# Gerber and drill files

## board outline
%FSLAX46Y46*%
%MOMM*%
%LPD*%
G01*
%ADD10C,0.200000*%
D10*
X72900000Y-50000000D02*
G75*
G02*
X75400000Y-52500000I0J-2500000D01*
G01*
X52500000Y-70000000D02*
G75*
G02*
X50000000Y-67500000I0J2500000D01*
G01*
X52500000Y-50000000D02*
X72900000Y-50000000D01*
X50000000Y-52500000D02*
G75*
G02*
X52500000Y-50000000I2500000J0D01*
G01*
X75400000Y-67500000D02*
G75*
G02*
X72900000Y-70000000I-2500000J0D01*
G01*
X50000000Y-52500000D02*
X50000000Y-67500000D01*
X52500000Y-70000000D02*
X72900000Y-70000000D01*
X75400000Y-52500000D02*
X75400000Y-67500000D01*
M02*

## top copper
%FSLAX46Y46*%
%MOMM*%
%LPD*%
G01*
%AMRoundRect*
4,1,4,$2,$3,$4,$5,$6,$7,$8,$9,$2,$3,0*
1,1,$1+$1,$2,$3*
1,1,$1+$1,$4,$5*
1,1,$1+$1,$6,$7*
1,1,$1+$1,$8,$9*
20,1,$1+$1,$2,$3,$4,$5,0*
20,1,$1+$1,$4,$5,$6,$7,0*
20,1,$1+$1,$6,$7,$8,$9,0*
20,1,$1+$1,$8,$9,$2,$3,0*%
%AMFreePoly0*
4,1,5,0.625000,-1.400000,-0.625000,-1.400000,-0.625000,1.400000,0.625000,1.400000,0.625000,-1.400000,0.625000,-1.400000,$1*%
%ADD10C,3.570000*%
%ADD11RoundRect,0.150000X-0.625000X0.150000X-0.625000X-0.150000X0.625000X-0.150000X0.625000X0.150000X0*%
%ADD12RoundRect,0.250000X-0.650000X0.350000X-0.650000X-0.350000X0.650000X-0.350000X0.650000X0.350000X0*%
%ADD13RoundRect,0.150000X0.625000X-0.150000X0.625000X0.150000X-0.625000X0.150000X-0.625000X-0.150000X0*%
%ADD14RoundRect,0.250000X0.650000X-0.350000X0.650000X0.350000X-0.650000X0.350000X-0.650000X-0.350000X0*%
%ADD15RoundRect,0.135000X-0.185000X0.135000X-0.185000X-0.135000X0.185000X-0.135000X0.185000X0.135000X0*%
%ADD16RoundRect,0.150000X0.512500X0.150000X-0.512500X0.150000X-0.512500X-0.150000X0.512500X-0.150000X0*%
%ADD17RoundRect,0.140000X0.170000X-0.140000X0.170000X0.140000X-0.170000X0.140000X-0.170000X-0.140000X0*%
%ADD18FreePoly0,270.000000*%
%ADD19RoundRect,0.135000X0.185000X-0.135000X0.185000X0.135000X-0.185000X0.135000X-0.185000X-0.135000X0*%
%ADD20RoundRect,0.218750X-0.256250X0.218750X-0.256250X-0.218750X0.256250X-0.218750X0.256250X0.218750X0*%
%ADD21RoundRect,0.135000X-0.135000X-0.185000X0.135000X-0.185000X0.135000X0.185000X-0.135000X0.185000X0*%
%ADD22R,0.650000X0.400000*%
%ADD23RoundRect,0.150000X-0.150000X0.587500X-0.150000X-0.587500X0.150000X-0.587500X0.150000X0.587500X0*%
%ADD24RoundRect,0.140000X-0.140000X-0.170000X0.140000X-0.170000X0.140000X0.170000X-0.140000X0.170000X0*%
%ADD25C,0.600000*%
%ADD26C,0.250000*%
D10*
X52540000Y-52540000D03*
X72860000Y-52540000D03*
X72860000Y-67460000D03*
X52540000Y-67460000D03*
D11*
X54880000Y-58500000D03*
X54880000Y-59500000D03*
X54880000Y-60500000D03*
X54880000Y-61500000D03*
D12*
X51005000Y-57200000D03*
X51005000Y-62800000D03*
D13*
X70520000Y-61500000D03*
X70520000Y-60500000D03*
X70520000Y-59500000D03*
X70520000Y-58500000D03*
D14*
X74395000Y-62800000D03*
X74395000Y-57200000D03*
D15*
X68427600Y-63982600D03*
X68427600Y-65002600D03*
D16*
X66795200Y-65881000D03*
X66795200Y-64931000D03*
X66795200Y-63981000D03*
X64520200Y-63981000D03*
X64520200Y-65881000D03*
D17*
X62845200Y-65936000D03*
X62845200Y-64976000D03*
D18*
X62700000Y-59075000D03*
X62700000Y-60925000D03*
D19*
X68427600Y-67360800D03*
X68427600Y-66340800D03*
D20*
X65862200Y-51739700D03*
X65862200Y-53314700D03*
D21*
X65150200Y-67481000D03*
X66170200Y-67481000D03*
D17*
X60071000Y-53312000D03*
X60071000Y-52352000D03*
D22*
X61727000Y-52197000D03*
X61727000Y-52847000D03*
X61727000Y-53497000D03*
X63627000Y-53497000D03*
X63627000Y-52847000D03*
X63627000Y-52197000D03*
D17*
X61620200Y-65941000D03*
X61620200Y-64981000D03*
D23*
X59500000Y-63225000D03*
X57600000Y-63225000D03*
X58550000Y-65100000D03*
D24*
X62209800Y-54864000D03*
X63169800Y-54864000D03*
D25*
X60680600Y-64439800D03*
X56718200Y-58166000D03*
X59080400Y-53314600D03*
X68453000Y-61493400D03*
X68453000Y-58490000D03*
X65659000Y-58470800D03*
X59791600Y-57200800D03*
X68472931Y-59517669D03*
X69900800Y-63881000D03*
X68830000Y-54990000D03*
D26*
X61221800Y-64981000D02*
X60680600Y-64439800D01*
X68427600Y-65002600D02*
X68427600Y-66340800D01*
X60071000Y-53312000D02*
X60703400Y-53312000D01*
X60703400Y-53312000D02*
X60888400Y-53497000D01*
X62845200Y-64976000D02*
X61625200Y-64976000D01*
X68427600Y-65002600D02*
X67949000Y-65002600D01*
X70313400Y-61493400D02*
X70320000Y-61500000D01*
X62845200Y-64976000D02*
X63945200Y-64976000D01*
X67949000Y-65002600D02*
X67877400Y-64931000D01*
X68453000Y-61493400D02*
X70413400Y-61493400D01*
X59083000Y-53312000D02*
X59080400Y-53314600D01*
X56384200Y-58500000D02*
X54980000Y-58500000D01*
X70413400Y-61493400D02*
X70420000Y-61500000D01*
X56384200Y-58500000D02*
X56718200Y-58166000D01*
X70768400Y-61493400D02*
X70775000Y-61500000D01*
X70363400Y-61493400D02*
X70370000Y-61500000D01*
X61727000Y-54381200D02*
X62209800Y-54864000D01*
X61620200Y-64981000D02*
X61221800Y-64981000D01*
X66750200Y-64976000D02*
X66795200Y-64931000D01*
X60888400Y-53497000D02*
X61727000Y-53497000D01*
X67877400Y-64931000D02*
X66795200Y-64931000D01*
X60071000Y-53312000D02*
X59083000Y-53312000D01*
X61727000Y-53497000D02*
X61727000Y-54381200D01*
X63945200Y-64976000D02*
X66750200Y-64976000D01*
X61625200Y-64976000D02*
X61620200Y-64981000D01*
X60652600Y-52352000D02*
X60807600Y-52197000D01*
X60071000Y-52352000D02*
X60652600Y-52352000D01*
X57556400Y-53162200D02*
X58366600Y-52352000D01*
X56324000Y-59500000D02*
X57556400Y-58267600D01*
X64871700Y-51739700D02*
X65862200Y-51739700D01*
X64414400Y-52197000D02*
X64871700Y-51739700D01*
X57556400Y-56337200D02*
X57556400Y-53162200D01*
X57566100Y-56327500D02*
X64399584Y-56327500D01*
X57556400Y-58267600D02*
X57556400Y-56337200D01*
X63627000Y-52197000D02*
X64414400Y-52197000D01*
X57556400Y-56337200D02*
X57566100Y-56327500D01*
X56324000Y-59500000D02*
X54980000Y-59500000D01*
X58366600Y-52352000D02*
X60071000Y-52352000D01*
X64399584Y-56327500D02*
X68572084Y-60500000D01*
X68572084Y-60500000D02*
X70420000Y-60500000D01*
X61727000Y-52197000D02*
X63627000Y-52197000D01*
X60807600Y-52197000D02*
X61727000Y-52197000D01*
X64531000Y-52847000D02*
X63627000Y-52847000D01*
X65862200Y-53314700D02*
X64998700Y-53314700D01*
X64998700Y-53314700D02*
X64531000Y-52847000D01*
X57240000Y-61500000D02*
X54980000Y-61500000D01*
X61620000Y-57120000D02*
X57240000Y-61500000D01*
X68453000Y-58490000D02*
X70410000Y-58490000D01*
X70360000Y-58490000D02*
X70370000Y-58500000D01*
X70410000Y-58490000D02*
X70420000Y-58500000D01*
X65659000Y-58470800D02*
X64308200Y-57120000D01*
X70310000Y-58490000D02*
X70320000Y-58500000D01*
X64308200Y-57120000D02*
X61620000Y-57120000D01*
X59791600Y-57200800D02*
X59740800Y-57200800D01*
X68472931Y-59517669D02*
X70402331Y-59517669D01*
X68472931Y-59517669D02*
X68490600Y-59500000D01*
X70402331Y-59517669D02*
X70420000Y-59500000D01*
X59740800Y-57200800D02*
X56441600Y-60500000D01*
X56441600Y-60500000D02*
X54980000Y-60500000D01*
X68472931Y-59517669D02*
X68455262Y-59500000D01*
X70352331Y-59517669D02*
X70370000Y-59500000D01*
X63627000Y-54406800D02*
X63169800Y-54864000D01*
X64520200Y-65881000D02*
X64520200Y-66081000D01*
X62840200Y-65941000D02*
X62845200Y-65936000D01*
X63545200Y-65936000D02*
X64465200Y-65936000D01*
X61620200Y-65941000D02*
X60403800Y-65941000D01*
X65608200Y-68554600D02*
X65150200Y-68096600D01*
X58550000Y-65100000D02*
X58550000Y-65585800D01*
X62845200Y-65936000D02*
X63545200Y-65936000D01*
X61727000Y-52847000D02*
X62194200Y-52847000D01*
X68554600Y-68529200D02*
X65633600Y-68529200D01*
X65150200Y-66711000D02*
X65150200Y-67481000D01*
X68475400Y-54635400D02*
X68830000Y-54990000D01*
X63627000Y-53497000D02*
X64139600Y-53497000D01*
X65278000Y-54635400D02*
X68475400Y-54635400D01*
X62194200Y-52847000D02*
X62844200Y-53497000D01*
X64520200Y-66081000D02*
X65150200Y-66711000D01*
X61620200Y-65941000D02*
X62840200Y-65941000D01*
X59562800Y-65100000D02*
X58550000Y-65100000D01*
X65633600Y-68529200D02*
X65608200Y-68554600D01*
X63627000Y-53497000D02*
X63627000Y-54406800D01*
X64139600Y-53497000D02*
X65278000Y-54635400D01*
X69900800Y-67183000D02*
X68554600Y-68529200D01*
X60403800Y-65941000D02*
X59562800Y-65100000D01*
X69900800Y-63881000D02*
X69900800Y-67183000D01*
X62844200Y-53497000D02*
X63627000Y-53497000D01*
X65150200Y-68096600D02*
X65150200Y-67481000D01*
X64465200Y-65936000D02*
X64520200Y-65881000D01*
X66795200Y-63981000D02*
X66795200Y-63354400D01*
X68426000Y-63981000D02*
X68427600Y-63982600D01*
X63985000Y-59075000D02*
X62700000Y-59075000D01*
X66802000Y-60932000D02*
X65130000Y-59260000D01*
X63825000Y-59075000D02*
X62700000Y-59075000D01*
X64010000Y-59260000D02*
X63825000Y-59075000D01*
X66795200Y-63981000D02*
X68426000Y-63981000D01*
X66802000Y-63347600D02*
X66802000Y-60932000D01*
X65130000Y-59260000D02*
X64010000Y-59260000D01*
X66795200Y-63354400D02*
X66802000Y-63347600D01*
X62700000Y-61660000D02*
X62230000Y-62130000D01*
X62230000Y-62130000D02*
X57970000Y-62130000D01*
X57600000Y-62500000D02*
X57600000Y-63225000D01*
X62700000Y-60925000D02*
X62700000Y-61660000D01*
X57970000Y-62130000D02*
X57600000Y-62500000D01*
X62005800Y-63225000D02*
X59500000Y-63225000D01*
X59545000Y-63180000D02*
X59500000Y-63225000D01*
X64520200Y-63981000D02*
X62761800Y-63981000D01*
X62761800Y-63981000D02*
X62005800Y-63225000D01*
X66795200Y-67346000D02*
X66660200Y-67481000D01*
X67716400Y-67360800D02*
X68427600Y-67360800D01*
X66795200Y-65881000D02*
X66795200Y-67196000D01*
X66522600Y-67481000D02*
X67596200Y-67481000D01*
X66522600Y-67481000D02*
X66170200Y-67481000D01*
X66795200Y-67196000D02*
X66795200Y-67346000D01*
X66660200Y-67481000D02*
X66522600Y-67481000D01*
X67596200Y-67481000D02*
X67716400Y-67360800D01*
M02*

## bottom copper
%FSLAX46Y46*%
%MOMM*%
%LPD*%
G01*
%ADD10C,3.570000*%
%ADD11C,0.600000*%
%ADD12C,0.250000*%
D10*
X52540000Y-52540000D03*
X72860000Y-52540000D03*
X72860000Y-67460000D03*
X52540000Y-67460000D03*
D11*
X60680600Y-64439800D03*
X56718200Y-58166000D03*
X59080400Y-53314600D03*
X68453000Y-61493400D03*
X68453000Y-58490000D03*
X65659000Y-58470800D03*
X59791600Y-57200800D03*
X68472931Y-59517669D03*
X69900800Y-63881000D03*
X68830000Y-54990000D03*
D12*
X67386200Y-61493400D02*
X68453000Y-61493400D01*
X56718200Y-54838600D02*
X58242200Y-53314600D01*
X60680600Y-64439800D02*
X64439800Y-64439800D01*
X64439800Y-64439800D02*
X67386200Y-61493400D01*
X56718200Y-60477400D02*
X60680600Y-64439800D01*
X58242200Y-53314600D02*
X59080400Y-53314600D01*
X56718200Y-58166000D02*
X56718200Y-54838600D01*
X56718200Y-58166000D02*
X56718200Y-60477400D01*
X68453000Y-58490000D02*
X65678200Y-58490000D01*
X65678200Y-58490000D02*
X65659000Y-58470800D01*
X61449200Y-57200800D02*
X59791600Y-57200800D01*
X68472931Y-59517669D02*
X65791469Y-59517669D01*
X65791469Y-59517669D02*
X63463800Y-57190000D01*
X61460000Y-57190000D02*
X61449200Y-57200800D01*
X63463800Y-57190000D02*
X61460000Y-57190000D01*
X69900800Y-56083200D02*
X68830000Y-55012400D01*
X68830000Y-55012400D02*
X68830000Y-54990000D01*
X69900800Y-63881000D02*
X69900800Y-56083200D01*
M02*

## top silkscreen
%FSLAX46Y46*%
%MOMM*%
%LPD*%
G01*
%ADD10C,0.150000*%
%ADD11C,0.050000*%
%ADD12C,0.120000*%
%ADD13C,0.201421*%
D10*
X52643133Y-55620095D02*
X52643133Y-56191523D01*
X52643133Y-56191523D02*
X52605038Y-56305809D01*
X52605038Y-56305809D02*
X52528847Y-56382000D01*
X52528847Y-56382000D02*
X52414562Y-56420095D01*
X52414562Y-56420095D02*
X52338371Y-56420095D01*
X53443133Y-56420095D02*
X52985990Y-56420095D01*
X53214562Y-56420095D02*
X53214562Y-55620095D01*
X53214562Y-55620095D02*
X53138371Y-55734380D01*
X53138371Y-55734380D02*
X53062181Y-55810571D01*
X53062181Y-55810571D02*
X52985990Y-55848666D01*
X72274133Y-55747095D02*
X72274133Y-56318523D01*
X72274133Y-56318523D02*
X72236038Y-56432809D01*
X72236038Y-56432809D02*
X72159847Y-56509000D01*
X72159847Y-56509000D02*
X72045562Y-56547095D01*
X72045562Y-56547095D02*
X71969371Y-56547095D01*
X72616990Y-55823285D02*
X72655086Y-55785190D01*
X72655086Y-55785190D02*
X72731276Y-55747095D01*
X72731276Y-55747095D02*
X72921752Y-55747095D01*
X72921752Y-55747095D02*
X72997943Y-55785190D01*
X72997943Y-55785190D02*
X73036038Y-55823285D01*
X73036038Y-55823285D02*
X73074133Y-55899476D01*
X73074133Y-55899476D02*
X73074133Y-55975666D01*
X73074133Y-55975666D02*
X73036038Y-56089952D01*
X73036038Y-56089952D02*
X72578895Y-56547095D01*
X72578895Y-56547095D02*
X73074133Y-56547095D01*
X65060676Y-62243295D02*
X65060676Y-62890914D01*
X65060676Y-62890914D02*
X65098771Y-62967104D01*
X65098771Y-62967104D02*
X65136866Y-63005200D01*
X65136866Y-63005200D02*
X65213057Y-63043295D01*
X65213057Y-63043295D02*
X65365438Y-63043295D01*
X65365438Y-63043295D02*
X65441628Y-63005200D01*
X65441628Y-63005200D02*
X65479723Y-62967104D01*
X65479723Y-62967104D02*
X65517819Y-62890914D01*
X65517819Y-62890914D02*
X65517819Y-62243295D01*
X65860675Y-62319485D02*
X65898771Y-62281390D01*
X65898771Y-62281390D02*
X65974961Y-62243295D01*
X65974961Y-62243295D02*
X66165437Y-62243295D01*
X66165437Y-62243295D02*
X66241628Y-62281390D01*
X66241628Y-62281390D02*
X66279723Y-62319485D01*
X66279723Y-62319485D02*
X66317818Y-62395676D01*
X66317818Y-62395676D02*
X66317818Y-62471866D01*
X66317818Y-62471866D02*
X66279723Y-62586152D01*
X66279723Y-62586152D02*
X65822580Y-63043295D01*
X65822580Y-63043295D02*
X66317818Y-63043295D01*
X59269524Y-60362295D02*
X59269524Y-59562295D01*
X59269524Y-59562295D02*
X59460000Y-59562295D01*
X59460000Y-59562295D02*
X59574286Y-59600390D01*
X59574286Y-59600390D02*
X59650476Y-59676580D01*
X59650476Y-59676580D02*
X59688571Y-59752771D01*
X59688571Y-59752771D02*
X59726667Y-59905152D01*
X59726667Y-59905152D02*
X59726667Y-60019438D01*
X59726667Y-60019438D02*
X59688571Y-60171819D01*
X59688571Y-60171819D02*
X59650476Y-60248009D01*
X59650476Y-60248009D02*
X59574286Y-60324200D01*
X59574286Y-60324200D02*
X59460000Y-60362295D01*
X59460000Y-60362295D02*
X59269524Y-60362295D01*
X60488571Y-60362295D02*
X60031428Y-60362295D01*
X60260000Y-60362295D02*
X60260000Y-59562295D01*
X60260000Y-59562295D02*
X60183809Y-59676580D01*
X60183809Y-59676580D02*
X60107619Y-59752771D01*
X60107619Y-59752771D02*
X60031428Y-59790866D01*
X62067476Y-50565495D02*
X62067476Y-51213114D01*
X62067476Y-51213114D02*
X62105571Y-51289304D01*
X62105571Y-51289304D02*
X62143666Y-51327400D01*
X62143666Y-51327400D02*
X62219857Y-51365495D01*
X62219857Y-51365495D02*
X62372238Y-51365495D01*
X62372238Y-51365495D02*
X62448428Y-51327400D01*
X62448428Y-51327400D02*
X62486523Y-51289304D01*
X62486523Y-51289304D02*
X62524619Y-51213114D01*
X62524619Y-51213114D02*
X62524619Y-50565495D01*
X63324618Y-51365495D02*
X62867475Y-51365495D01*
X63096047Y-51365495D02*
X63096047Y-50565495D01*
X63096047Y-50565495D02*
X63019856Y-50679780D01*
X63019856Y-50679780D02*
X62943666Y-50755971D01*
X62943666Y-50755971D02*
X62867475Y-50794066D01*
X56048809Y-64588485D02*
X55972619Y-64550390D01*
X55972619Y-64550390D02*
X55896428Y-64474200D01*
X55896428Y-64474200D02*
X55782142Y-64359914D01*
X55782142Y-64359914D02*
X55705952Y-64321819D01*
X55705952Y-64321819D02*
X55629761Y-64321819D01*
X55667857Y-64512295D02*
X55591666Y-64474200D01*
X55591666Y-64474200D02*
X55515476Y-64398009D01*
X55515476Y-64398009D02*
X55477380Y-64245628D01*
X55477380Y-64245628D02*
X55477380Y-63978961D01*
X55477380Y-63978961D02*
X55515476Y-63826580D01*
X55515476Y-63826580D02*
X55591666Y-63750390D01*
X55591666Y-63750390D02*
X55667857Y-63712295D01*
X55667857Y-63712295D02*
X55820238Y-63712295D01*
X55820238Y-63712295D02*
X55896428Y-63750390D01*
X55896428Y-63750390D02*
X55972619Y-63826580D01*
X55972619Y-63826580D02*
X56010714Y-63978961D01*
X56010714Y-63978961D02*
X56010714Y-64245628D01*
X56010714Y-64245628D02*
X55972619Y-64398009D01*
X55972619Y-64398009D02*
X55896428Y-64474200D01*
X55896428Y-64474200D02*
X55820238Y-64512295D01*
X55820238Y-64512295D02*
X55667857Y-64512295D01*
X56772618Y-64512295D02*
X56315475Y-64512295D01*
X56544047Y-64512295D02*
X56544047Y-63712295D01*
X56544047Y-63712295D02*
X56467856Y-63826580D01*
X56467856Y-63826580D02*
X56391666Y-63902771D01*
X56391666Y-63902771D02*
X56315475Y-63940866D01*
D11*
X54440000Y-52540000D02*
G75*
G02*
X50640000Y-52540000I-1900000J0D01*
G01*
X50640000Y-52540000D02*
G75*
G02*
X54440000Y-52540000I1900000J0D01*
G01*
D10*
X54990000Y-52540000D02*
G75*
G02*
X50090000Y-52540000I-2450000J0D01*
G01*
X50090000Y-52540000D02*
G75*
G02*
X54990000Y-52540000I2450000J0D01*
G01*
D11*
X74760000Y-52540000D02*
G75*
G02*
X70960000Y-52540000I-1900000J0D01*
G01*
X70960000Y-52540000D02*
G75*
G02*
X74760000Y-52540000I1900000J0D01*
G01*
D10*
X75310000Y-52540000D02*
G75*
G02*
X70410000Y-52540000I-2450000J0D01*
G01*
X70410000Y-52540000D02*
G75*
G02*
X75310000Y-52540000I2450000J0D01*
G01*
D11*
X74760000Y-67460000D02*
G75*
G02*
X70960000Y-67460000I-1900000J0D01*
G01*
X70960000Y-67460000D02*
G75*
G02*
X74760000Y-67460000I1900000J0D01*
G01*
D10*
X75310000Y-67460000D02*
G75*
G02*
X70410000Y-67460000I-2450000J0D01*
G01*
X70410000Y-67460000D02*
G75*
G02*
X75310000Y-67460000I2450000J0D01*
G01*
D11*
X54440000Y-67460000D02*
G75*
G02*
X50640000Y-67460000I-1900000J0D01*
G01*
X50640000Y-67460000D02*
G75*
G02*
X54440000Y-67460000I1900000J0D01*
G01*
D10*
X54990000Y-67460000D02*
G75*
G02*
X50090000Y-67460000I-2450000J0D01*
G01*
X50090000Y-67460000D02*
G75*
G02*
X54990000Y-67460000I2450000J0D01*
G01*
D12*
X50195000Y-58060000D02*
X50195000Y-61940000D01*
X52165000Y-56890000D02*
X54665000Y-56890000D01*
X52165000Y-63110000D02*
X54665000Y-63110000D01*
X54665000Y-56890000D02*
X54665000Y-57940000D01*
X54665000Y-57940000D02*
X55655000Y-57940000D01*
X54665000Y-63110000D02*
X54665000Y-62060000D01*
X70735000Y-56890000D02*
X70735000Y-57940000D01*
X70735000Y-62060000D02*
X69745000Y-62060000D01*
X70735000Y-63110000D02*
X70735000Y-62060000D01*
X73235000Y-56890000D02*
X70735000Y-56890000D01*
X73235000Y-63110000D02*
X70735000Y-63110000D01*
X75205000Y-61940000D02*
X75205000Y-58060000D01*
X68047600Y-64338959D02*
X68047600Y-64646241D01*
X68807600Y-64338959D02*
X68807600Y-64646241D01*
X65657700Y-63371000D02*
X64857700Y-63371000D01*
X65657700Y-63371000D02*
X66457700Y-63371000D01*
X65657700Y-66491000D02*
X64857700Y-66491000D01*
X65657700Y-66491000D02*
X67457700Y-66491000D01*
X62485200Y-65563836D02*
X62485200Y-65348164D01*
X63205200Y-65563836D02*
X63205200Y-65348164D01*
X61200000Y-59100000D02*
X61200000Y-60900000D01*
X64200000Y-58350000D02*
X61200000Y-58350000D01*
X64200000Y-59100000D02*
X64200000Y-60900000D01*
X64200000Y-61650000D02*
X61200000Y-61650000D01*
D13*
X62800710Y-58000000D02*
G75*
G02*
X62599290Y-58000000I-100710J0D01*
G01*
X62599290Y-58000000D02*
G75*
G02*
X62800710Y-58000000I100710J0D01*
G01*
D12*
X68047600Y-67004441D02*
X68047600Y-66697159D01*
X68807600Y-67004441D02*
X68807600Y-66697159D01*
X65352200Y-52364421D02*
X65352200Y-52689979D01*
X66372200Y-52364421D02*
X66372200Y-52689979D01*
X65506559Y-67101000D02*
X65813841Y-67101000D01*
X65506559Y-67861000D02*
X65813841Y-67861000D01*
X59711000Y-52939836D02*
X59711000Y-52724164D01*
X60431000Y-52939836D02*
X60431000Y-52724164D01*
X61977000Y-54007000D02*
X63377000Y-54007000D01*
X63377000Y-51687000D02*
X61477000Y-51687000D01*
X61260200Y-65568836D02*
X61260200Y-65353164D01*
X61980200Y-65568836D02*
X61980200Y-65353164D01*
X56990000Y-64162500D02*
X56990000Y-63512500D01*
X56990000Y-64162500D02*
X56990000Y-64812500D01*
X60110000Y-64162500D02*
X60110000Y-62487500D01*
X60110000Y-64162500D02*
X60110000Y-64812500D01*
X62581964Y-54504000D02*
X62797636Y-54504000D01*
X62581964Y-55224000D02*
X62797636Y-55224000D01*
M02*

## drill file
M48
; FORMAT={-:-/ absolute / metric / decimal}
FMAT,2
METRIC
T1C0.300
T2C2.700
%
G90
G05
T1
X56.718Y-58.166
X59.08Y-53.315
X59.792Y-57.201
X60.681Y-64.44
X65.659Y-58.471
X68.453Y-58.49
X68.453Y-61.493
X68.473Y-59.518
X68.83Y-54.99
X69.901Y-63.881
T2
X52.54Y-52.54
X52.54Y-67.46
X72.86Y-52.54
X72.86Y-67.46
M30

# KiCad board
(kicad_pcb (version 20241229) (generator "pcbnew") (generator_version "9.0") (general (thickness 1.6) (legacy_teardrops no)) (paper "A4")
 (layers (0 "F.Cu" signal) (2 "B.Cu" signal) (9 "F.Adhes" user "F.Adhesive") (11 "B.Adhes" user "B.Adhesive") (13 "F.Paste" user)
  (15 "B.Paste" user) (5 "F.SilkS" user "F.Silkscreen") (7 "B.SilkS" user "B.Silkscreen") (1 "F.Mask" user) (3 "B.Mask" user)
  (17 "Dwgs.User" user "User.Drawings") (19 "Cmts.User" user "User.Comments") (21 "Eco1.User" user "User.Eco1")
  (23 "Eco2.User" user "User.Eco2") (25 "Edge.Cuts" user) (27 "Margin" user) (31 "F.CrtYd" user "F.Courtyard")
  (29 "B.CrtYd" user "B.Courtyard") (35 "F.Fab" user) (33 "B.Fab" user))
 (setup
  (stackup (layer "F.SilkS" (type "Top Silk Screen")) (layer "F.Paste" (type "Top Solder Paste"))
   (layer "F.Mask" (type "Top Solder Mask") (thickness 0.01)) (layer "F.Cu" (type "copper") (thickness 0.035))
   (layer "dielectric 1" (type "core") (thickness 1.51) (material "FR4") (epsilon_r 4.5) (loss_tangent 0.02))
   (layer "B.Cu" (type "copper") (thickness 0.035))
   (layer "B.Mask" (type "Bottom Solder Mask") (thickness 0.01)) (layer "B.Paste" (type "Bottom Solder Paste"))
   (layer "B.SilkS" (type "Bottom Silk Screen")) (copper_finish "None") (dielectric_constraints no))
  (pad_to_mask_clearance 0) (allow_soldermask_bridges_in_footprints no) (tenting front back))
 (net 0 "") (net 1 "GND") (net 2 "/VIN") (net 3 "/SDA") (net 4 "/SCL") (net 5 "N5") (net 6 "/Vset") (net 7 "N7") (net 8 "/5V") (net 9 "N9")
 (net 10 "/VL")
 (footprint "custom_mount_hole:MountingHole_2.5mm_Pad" (layer "F.Cu") (at 52.54 52.54)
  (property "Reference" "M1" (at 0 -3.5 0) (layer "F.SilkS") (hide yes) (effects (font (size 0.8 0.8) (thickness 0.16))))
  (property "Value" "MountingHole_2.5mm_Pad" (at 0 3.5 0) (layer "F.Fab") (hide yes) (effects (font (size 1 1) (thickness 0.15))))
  (fp_circle (center 0 0) (end 1.9 0) (stroke (width 0.05) (type solid)) (fill no) (layer "F.SilkS"))
  (fp_circle (center 0 0) (end 2.45 0) (stroke (width 0.15) (type solid)) (fill no) (layer "F.SilkS"))
  (pad "~" thru_hole circle (at 0 0) (size 3.57 3.57) (drill 2.7) (layers "*.Cu" "*.Mask") (remove_unused_layers no)))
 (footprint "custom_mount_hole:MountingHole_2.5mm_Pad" (layer "F.Cu") (at 72.86 52.54)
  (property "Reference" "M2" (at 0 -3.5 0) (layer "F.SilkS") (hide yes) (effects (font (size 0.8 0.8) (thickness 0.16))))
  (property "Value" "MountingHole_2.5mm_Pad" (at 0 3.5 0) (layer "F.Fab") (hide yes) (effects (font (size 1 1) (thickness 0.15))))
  (fp_circle (center 0 0) (end 1.9 0) (stroke (width 0.05) (type solid)) (fill no) (layer "F.SilkS"))
  (fp_circle (center 0 0) (end 2.45 0) (stroke (width 0.15) (type solid)) (fill no) (layer "F.SilkS"))
  (pad "~" thru_hole circle (at 0 0) (size 3.57 3.57) (drill 2.7) (layers "*.Cu" "*.Mask") (remove_unused_layers no)))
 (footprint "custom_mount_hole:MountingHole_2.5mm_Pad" (layer "F.Cu") (at 72.86 67.46)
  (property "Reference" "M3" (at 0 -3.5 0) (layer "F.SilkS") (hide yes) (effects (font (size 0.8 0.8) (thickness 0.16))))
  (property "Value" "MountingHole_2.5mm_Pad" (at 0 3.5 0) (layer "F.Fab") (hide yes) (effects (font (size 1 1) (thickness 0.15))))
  (fp_circle (center 0 0) (end 1.9 0) (stroke (width 0.05) (type solid)) (fill no) (layer "F.SilkS"))
  (fp_circle (center 0 0) (end 2.45 0) (stroke (width 0.15) (type solid)) (fill no) (layer "F.SilkS"))
  (pad "~" thru_hole circle (at 0 0) (size 3.57 3.57) (drill 2.7) (layers "*.Cu" "*.Mask") (remove_unused_layers no)))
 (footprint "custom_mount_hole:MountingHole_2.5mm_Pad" (layer "F.Cu") (at 52.54 67.46)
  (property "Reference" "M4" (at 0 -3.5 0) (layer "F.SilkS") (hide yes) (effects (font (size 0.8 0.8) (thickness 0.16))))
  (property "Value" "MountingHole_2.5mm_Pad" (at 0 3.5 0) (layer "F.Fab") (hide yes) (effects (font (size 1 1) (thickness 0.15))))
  (fp_circle (center 0 0) (end 1.9 0) (stroke (width 0.05) (type solid)) (fill no) (layer "F.SilkS"))
  (fp_circle (center 0 0) (end 2.45 0) (stroke (width 0.15) (type solid)) (fill no) (layer "F.SilkS"))
  (pad "~" thru_hole circle (at 0 0) (size 3.57 3.57) (drill 2.7) (layers "*.Cu" "*.Mask") (remove_unused_layers no)))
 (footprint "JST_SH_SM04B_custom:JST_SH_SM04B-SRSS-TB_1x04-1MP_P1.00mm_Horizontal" (layer "F.Cu") (at 52.88 60 -90)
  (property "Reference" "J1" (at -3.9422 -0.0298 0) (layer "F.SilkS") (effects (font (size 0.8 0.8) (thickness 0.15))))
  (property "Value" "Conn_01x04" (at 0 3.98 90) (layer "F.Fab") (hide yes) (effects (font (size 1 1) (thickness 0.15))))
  (fp_line (start -1.94 2.685) (end 1.94 2.685) (stroke (width 0.12) (type solid)) (layer "F.SilkS"))
  (fp_line (start -3.11 0.715) (end -3.11 -1.785) (stroke (width 0.12) (type solid)) (layer "F.SilkS"))
  (fp_line (start 3.11 0.715) (end 3.11 -1.785) (stroke (width 0.12) (type solid)) (layer "F.SilkS"))
  (fp_line (start -3.11 -1.785) (end -2.06 -1.785) (stroke (width 0.12) (type solid)) (layer "F.SilkS"))
  (fp_line (start -2.06 -1.785) (end -2.06 -2.775) (stroke (width 0.12) (type solid)) (layer "F.SilkS"))
  (fp_line (start 3.11 -1.785) (end 2.06 -1.785) (stroke (width 0.12) (type solid)) (layer "F.SilkS"))
  (pad "1" smd roundrect (at -1.5 -2 270) (size 0.6 1.55) (layers "F.Cu" "F.Mask" "F.Paste") (roundrect_rratio 0.25) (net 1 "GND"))
  (pad "2" smd roundrect (at -0.5 -2 270) (size 0.6 1.55) (layers "F.Cu" "F.Mask" "F.Paste") (roundrect_rratio 0.25) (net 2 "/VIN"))
  (pad "3" smd roundrect (at 0.5 -2 270) (size 0.6 1.55) (layers "F.Cu" "F.Mask" "F.Paste") (roundrect_rratio 0.25) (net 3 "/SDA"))
  (pad "4" smd roundrect (at 1.5 -2 270) (size 0.6 1.55) (layers "F.Cu" "F.Mask" "F.Paste") (roundrect_rratio 0.25) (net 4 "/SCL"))
  (pad "MP" smd roundrect (at -2.8 1.875 270) (size 1.2 1.8) (layers "F.Cu" "F.Mask" "F.Paste") (roundrect_rratio 0.2083333333))
  (pad "MP" smd roundrect (at 2.8 1.875 270) (size 1.2 1.8) (layers "F.Cu" "F.Mask" "F.Paste") (roundrect_rratio 0.2083333333)))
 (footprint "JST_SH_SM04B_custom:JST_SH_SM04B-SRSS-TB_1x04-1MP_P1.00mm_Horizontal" (layer "F.Cu") (at 72.52 60 90)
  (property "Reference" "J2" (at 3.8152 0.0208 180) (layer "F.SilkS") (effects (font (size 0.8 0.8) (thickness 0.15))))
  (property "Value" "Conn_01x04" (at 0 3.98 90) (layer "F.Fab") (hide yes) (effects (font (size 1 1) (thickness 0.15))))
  (fp_line (start 3.11 -1.785) (end 2.06 -1.785) (stroke (width 0.12) (type solid)) (layer "F.SilkS"))
  (fp_line (start -2.06 -1.785) (end -2.06 -2.775) (stroke (width 0.12) (type solid)) (layer "F.SilkS"))
  (fp_line (start -3.11 -1.785) (end -2.06 -1.785) (stroke (width 0.12) (type solid)) (layer "F.SilkS"))
  (fp_line (start 3.11 0.715) (end 3.11 -1.785) (stroke (width 0.12) (type solid)) (layer "F.SilkS"))
  (fp_line (start -3.11 0.715) (end -3.11 -1.785) (stroke (width 0.12) (type solid)) (layer "F.SilkS"))
  (fp_line (start -1.94 2.685) (end 1.94 2.685) (stroke (width 0.12) (type solid)) (layer "F.SilkS"))
  (pad "1" smd roundrect (at -1.5 -2 90) (size 0.6 1.55) (layers "F.Cu" "F.Mask" "F.Paste") (roundrect_rratio 0.25) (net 1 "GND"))
  (pad "2" smd roundrect (at -0.5 -2 90) (size 0.6 1.55) (layers "F.Cu" "F.Mask" "F.Paste") (roundrect_rratio 0.25) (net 2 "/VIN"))
  (pad "3" smd roundrect (at 0.5 -2 90) (size 0.6 1.55) (layers "F.Cu" "F.Mask" "F.Paste") (roundrect_rratio 0.25) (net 3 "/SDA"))
  (pad "4" smd roundrect (at 1.5 -2 90) (size 0.6 1.55) (layers "F.Cu" "F.Mask" "F.Paste") (roundrect_rratio 0.25) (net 4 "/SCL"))
  (pad "MP" smd roundrect (at -2.8 1.875 90) (size 1.2 1.8) (layers "F.Cu" "F.Mask" "F.Paste") (roundrect_rratio 0.2083333333))
  (pad "MP" smd roundrect (at 2.8 1.875 90) (size 1.2 1.8) (layers "F.Cu" "F.Mask" "F.Paste") (roundrect_rratio 0.2083333333)))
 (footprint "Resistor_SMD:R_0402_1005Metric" (layer "F.Cu") (at 68.4276 64.4926 -90)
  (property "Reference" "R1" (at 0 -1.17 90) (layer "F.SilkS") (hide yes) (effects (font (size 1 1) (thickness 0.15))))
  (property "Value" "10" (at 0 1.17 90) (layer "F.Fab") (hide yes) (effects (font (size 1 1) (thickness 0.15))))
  (fp_line (start -0.153641 0.38) (end 0.153641 0.38) (stroke (width 0.12) (type solid)) (layer "F.SilkS"))
  (fp_line (start -0.153641 -0.38) (end 0.153641 -0.38) (stroke (width 0.12) (type solid)) (layer "F.SilkS"))
  (pad "1" smd roundrect (at -0.51 0 270) (size 0.54 0.64) (layers "F.Cu" "F.Mask" "F.Paste") (roundrect_rratio 0.25) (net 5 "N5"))
  (pad "2" smd roundrect (at 0.51 0 270) (size 0.54 0.64) (layers "F.Cu" "F.Mask" "F.Paste") (roundrect_rratio 0.25) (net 1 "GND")))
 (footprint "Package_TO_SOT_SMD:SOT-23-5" (layer "F.Cu") (at 65.6577 64.931 180)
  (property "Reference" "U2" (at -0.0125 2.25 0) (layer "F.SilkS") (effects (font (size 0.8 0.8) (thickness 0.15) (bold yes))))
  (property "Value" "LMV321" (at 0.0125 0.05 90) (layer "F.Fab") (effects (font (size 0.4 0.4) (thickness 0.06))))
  (fp_line (start 0 1.56) (end 0.8 1.56) (stroke (width 0.12) (type solid)) (layer "F.SilkS"))
  (fp_line (start 0 1.56) (end -0.8 1.56) (stroke (width 0.12) (type solid)) (layer "F.SilkS"))
  (fp_line (start 0 -1.56) (end 0.8 -1.56) (stroke (width 0.12) (type solid)) (layer "F.SilkS"))
  (fp_line (start 0 -1.56) (end -1.8 -1.56) (stroke (width 0.12) (type solid)) (layer "F.SilkS"))
  (pad "1" smd roundrect (at -1.1375 -0.95 180) (size 1.325 0.6) (layers "F.Cu" "F.Mask" "F.Paste") (roundrect_rratio 0.25) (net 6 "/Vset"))
  (pad "2" smd roundrect (at -1.1375 0 180) (size 1.325 0.6) (layers "F.Cu" "F.Mask" "F.Paste") (roundrect_rratio 0.25) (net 1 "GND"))
  (pad "3" smd roundrect (at -1.1375 0.95 180) (size 1.325 0.6) (layers "F.Cu" "F.Mask" "F.Paste") (roundrect_rratio 0.25) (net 5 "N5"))
  (pad "4" smd roundrect (at 1.1375 0.95 180) (size 1.325 0.6) (layers "F.Cu" "F.Mask" "F.Paste") (roundrect_rratio 0.25) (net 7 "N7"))
  (pad "5" smd roundrect (at 1.1375 -0.95 180) (size 1.325 0.6) (layers "F.Cu" "F.Mask" "F.Paste") (roundrect_rratio 0.25) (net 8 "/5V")))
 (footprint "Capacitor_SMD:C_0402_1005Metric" (layer "F.Cu") (at 62.8452 65.456 90)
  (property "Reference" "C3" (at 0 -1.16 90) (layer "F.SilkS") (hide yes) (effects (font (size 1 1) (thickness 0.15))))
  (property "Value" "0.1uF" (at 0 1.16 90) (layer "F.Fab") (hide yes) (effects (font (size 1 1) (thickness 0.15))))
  (fp_line (start -0.107836 -0.36) (end 0.107836 -0.36) (stroke (width 0.12) (type solid)) (layer "F.SilkS"))
  (fp_line (start -0.107836 0.36) (end 0.107836 0.36) (stroke (width 0.12) (type solid)) (layer "F.SilkS"))
  (pad "1" smd roundrect (at -0.48 0 90) (size 0.56 0.62) (layers "F.Cu" "F.Mask" "F.Paste") (roundrect_rratio 0.25) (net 8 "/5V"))
  (pad "2" smd roundrect (at 0.48 0 90) (size 0.56 0.62) (layers "F.Cu" "F.Mask" "F.Paste") (roundrect_rratio 0.25) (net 1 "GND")))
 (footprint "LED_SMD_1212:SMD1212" (layer "F.Cu") (at 62.7 60 -90)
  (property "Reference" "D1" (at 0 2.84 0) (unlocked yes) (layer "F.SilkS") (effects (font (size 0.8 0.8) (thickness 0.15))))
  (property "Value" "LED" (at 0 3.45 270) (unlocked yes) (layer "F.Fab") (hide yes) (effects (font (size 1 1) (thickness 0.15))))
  (fp_line (start -0.9 1.5) (end 0.9 1.5) (stroke (width 0.12) (type default)) (layer "F.SilkS"))
  (fp_line (start -1.65 -1.5) (end -1.65 1.5) (stroke (width 0.12) (type default)) (layer "F.SilkS"))
  (fp_line (start -0.9 -1.5) (end 0.9 -1.5) (stroke (width 0.12) (type default)) (layer "F.SilkS"))
  (fp_line (start 1.65 -1.5) (end 1.65 1.5) (stroke (width 0.12) (type default)) (layer "F.SilkS"))
  (fp_circle (center -2 0) (end -1.9 0.1) (stroke (width 0.12) (type solid)) (fill yes) (layer "F.SilkS"))
  (pad "1" smd custom (at -0.925 0 270) (size 1.25 2.8) (layers "F.Cu" "F.Mask" "F.Paste") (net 5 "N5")
   (options (clearance outline) (anchor rect)) (primitives))
  (pad "2" smd custom (at 0.925 0 270) (size 1.25 2.8) (layers "F.Cu" "F.Mask" "F.Paste") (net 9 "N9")
   (options (clearance outline) (anchor rect)) (primitives)))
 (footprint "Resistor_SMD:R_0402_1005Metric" (layer "F.Cu") (at 68.4276 66.8508 90)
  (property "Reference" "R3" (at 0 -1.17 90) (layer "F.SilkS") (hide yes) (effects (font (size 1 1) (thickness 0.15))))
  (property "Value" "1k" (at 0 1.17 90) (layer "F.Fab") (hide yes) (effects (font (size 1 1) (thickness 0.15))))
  (fp_line (start -0.153641 -0.38) (end 0.153641 -0.38) (stroke (width 0.12) (type solid)) (layer "F.SilkS"))
  (fp_line (start -0.153641 0.38) (end 0.153641 0.38) (stroke (width 0.12) (type solid)) (layer "F.SilkS"))
  (pad "1" smd roundrect (at -0.51 0 90) (size 0.54 0.64) (layers "F.Cu" "F.Mask" "F.Paste") (roundrect_rratio 0.25) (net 6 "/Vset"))
  (pad "2" smd roundrect (at 0.51 0 90) (size 0.54 0.64) (layers "F.Cu" "F.Mask" "F.Paste") (roundrect_rratio 0.25) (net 1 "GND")))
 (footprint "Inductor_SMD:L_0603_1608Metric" (layer "F.Cu") (at 65.8622 52.5272 -90)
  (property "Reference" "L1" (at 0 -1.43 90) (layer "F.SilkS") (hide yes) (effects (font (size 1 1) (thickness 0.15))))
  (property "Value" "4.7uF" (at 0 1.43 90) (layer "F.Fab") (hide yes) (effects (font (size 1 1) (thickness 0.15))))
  (fp_line (start -0.162779 0.51) (end 0.162779 0.51) (stroke (width 0.12) (type solid)) (layer "F.SilkS"))
  (fp_line (start -0.162779 -0.51) (end 0.162779 -0.51) (stroke (width 0.12) (type solid)) (layer "F.SilkS"))
  (pad "1" smd roundrect (at -0.7875 0 270) (size 0.875 0.95) (layers "F.Cu" "F.Mask" "F.Paste") (roundrect_rratio 0.25) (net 2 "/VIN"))
  (pad "2" smd roundrect (at 0.7875 0 270) (size 0.875 0.95) (layers "F.Cu" "F.Mask" "F.Paste") (roundrect_rratio 0.25) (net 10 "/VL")))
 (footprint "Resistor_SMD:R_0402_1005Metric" (layer "F.Cu") (at 65.6602 67.481)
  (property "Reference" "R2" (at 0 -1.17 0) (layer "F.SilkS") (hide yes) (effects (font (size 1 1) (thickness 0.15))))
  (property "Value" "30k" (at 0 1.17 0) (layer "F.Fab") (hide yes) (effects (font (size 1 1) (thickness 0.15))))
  (fp_line (start -0.153641 -0.38) (end 0.153641 -0.38) (stroke (width 0.12) (type solid)) (layer "F.SilkS"))
  (fp_line (start -0.153641 0.38) (end 0.153641 0.38) (stroke (width 0.12) (type solid)) (layer "F.SilkS"))
  (pad "1" smd roundrect (at -0.51 0) (size 0.54 0.64) (layers "F.Cu" "F.Mask" "F.Paste") (roundrect_rratio 0.25) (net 8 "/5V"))
  (pad "2" smd roundrect (at 0.51 0) (size 0.54 0.64) (layers "F.Cu" "F.Mask" "F.Paste") (roundrect_rratio 0.25) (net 6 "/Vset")))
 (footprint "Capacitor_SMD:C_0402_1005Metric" (layer "F.Cu") (at 60.071 52.832 90)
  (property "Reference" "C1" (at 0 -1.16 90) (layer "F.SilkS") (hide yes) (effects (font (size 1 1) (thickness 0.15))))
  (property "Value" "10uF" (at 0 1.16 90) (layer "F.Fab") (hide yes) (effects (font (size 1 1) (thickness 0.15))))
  (fp_line (start -0.107836 -0.36) (end 0.107836 -0.36) (stroke (width 0.12) (type solid)) (layer "F.SilkS"))
  (fp_line (start -0.107836 0.36) (end 0.107836 0.36) (stroke (width 0.12) (type solid)) (layer "F.SilkS"))
  (pad "1" smd roundrect (at -0.48 0 90) (size 0.56 0.62) (layers "F.Cu" "F.Mask" "F.Paste") (roundrect_rratio 0.25) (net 1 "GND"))
  (pad "2" smd roundrect (at 0.48 0 90) (size 0.56 0.62) (layers "F.Cu" "F.Mask" "F.Paste") (roundrect_rratio 0.25) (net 2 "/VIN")))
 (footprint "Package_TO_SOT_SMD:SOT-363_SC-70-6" (layer "F.Cu") (at 62.677 52.847)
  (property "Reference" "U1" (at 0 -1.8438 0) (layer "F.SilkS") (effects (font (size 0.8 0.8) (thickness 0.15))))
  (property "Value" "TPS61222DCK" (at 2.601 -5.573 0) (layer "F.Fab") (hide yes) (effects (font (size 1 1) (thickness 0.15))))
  (fp_line (start -0.7 1.16) (end 0.7 1.16) (stroke (width 0.12) (type solid)) (layer "F.SilkS"))
  (fp_line (start 0.7 -1.16) (end -1.2 -1.16) (stroke (width 0.12) (type solid)) (layer "F.SilkS"))
  (pad "1" smd rect (at -0.95 -0.65) (size 0.65 0.4) (layers "F.Cu" "F.Mask" "F.Paste") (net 2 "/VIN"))
  (pad "2" smd rect (at -0.95 0) (size 0.65 0.4) (layers "F.Cu" "F.Mask" "F.Paste") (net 8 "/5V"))
  (pad "3" smd rect (at -0.95 0.65) (size 0.65 0.4) (layers "F.Cu" "F.Mask" "F.Paste") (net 1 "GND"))
  (pad "4" smd rect (at 0.95 0.65) (size 0.65 0.4) (layers "F.Cu" "F.Mask" "F.Paste") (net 8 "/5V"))
  (pad "5" smd rect (at 0.95 0) (size 0.65 0.4) (layers "F.Cu" "F.Mask" "F.Paste") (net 10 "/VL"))
  (pad "6" smd rect (at 0.95 -0.65) (size 0.65 0.4) (layers "F.Cu" "F.Mask" "F.Paste") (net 2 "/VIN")))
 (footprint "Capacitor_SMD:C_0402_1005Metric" (layer "F.Cu") (at 61.6202 65.461 90)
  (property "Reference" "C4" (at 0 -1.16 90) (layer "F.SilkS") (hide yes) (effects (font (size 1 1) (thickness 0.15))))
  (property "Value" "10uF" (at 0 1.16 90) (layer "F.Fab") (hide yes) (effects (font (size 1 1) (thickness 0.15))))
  (fp_line (start -0.107836 -0.36) (end 0.107836 -0.36) (stroke (width 0.12) (type solid)) (layer "F.SilkS"))
  (fp_line (start -0.107836 0.36) (end 0.107836 0.36) (stroke (width 0.12) (type solid)) (layer "F.SilkS"))
  (pad "1" smd roundrect (at -0.48 0 90) (size 0.56 0.62) (layers "F.Cu" "F.Mask" "F.Paste") (roundrect_rratio 0.25) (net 8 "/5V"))
  (pad "2" smd roundrect (at 0.48 0 90) (size 0.56 0.62) (layers "F.Cu" "F.Mask" "F.Paste") (roundrect_rratio 0.25) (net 1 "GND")))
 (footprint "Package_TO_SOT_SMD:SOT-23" (layer "F.Cu") (at 58.55 64.1625 -90)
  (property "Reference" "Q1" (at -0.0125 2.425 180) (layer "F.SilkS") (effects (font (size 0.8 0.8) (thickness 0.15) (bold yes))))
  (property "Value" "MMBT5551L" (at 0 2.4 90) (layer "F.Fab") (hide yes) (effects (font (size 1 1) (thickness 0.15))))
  (fp_line (start 0 1.56) (end -0.65 1.56) (stroke (width 0.12) (type solid)) (layer "F.SilkS"))
  (fp_line (start 0 1.56) (end 0.65 1.56) (stroke (width 0.12) (type solid)) (layer "F.SilkS"))
  (fp_line (start 0 -1.56) (end -1.675 -1.56) (stroke (width 0.12) (type solid)) (layer "F.SilkS"))
  (fp_line (start 0 -1.56) (end 0.65 -1.56) (stroke (width 0.12) (type solid)) (layer "F.SilkS"))
  (pad "1" smd roundrect (at -0.9375 -0.95 270) (size 1.475 0.6) (layers "F.Cu" "F.Mask" "F.Paste") (roundrect_rratio 0.25) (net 7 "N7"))
  (pad "2" smd roundrect (at -0.9375 0.95 270) (size 1.475 0.6) (layers "F.Cu" "F.Mask" "F.Paste") (roundrect_rratio 0.25) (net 9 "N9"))
  (pad "3" smd roundrect (at 0.9375 0 270) (size 1.475 0.6) (layers "F.Cu" "F.Mask" "F.Paste") (roundrect_rratio 0.25) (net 8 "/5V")))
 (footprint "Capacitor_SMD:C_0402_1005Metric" (layer "F.Cu") (at 62.6898 54.864)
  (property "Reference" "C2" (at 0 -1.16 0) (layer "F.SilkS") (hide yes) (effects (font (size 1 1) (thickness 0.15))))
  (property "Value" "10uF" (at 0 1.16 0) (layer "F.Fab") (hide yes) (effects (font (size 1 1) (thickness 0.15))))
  (fp_line (start -0.107836 -0.36) (end 0.107836 -0.36) (stroke (width 0.12) (type solid)) (layer "F.SilkS"))
  (fp_line (start -0.107836 0.36) (end 0.107836 0.36) (stroke (width 0.12) (type solid)) (layer "F.SilkS"))
  (pad "1" smd roundrect (at -0.48 0) (size 0.56 0.62) (layers "F.Cu" "F.Mask" "F.Paste") (roundrect_rratio 0.25) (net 1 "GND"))
  (pad "2" smd roundrect (at 0.48 0) (size 0.56 0.62) (layers "F.Cu" "F.Mask" "F.Paste") (roundrect_rratio 0.25) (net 8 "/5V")))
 (gr_arc (start 72.9 50) (mid 74.667767 50.732233) (end 75.4 52.5) (stroke (width 0.2) (type solid)) (layer "Edge.Cuts"))
 (gr_arc (start 52.5 70) (mid 50.732233 69.267767) (end 50 67.5) (stroke (width 0.2) (type solid)) (layer "Edge.Cuts"))
 (gr_line (start 52.5 50) (end 72.9 50) (stroke (width 0.2) (type solid)) (layer "Edge.Cuts"))
 (gr_arc (start 50 52.5) (mid 50.732233 50.732233) (end 52.5 50) (stroke (width 0.2) (type solid)) (layer "Edge.Cuts"))
 (gr_arc (start 75.4 67.5) (mid 74.667767 69.267767) (end 72.9 70) (stroke (width 0.2) (type solid)) (layer "Edge.Cuts"))
 (gr_line (start 50 52.5) (end 50 67.5) (stroke (width 0.2) (type solid)) (layer "Edge.Cuts"))
 (gr_line (start 52.5 70) (end 72.9 70) (stroke (width 0.2) (type solid)) (layer "Edge.Cuts"))
 (gr_line (start 75.4 52.5) (end 75.4 67.5) (stroke (width 0.2) (type solid)) (layer "Edge.Cuts"))
 (segment (start 61.2218 64.981) (end 60.6806 64.4398) (width 0.25) (layer "F.Cu") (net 1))
 (segment (start 68.4276 65.0026) (end 68.4276 66.3408) (width 0.25) (layer "F.Cu") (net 1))
 (segment (start 60.071 53.312) (end 60.7034 53.312) (width 0.25) (layer "F.Cu") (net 1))
 (segment (start 60.7034 53.312) (end 60.8884 53.497) (width 0.25) (layer "F.Cu") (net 1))
 (segment (start 62.8452 64.976) (end 61.6252 64.976) (width 0.25) (layer "F.Cu") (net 1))
 (segment (start 68.4276 65.0026) (end 67.949 65.0026) (width 0.25) (layer "F.Cu") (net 1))
 (segment (start 70.3134 61.4934) (end 70.32 61.5) (width 0.25) (layer "F.Cu") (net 1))
 (segment (start 62.8452 64.976) (end 63.9452 64.976) (width 0.25) (layer "F.Cu") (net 1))
 (segment (start 67.949 65.0026) (end 67.8774 64.931) (width 0.25) (layer "F.Cu") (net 1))
 (segment (start 68.453 61.4934) (end 70.4134 61.4934) (width 0.25) (layer "F.Cu") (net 1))
 (segment (start 59.083 53.312) (end 59.0804 53.3146) (width 0.25) (layer "F.Cu") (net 1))
 (segment (start 56.3842 58.5) (end 54.98 58.5) (width 0.25) (layer "F.Cu") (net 1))
 (segment (start 70.4134 61.4934) (end 70.42 61.5) (width 0.25) (layer "F.Cu") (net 1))
 (segment (start 56.3842 58.5) (end 56.7182 58.166) (width 0.25) (layer "F.Cu") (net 1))
 (segment (start 70.7684 61.4934) (end 70.775 61.5) (width 0.25) (layer "F.Cu") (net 1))
 (segment (start 70.3634 61.4934) (end 70.37 61.5) (width 0.25) (layer "F.Cu") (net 1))
 (segment (start 61.727 54.3812) (end 62.2098 54.864) (width 0.25) (layer "F.Cu") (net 1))
 (segment (start 61.6202 64.981) (end 61.2218 64.981) (width 0.25) (layer "F.Cu") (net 1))
 (segment (start 66.7502 64.976) (end 66.7952 64.931) (width 0.25) (layer "F.Cu") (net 1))
 (segment (start 60.8884 53.497) (end 61.727 53.497) (width 0.25) (layer "F.Cu") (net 1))
 (segment (start 67.8774 64.931) (end 66.7952 64.931) (width 0.25) (layer "F.Cu") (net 1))
 (segment (start 60.071 53.312) (end 59.083 53.312) (width 0.25) (layer "F.Cu") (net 1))
 (segment (start 61.727 53.497) (end 61.727 54.3812) (width 0.25) (layer "F.Cu") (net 1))
 (segment (start 63.9452 64.976) (end 66.7502 64.976) (width 0.25) (layer "F.Cu") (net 1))
 (segment (start 61.6252 64.976) (end 61.6202 64.981) (width 0.25) (layer "F.Cu") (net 1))
 (via (at 60.6806 64.4398) (size 0.6) (drill 0.3) (layers "F.Cu" "B.Cu") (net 1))
 (via (at 56.7182 58.166) (size 0.6) (drill 0.3) (layers "F.Cu" "B.Cu") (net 1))
 (via (at 59.0804 53.3146) (size 0.6) (drill 0.3) (layers "F.Cu" "B.Cu") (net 1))
 (via (at 68.453 61.4934) (size 0.6) (drill 0.3) (layers "F.Cu" "B.Cu") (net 1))
 (segment (start 67.3862 61.4934) (end 68.453 61.4934) (width 0.25) (layer "B.Cu") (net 1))
 (segment (start 56.7182 54.8386) (end 58.2422 53.3146) (width 0.25) (layer "B.Cu") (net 1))
 (segment (start 60.6806 64.4398) (end 64.4398 64.4398) (width 0.25) (layer "B.Cu") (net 1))
 (segment (start 64.4398 64.4398) (end 67.3862 61.4934) (width 0.25) (layer "B.Cu") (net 1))
 (segment (start 56.7182 60.4774) (end 60.6806 64.4398) (width 0.25) (layer "B.Cu") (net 1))
 (segment (start 58.2422 53.3146) (end 59.0804 53.3146) (width 0.25) (layer "B.Cu") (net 1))
 (segment (start 56.7182 58.166) (end 56.7182 54.8386) (width 0.25) (layer "B.Cu") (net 1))
 (segment (start 56.7182 58.166) (end 56.7182 60.4774) (width 0.25) (layer "B.Cu") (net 1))
 (segment (start 60.6526 52.352) (end 60.8076 52.197) (width 0.25) (layer "F.Cu") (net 2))
 (segment (start 60.071 52.352) (end 60.6526 52.352) (width 0.25) (layer "F.Cu") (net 2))
 (segment (start 57.5564 53.1622) (end 58.3666 52.352) (width 0.25) (layer "F.Cu") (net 2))
 (segment (start 56.324 59.5) (end 57.5564 58.2676) (width 0.25) (layer "F.Cu") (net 2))
 (segment (start 64.8717 51.7397) (end 65.8622 51.7397) (width 0.25) (layer "F.Cu") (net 2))
 (segment (start 64.4144 52.197) (end 64.8717 51.7397) (width 0.25) (layer "F.Cu") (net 2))
 (segment (start 57.5564 56.3372) (end 57.5564 53.1622) (width 0.25) (layer "F.Cu") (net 2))
 (segment (start 57.5661 56.3275) (end 64.399584 56.3275) (width 0.25) (layer "F.Cu") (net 2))
 (segment (start 57.5564 58.2676) (end 57.5564 56.3372) (width 0.25) (layer "F.Cu") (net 2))
 (segment (start 63.627 52.197) (end 64.4144 52.197) (width 0.25) (layer "F.Cu") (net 2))
 (segment (start 57.5564 56.3372) (end 57.5661 56.3275) (width 0.25) (layer "F.Cu") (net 2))
 (segment (start 56.324 59.5) (end 54.98 59.5) (width 0.25) (layer "F.Cu") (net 2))
 (segment (start 58.3666 52.352) (end 60.071 52.352) (width 0.25) (layer "F.Cu") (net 2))
 (segment (start 64.399584 56.3275) (end 68.572084 60.5) (width 0.25) (layer "F.Cu") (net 2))
 (segment (start 68.572084 60.5) (end 70.42 60.5) (width 0.25) (layer "F.Cu") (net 2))
 (segment (start 61.727 52.197) (end 63.627 52.197) (width 0.25) (layer "F.Cu") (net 2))
 (segment (start 60.8076 52.197) (end 61.727 52.197) (width 0.25) (layer "F.Cu") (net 2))
 (segment (start 64.531 52.847) (end 63.627 52.847) (width 0.25) (layer "F.Cu") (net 10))
 (segment (start 65.8622 53.3147) (end 64.9987 53.3147) (width 0.25) (layer "F.Cu") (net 10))
 (segment (start 64.9987 53.3147) (end 64.531 52.847) (width 0.25) (layer "F.Cu") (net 10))
 (segment (start 57.24 61.5) (end 54.98 61.5) (width 0.25) (layer "F.Cu") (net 4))
 (segment (start 61.62 57.12) (end 57.24 61.5) (width 0.25) (layer "F.Cu") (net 4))
 (segment (start 68.453 58.49) (end 70.41 58.49) (width 0.25) (layer "F.Cu") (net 4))
 (segment (start 70.36 58.49) (end 70.37 58.5) (width 0.25) (layer "F.Cu") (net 4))
 (segment (start 70.41 58.49) (end 70.42 58.5) (width 0.25) (layer "F.Cu") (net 4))
 (segment (start 65.659 58.4708) (end 64.3082 57.12) (width 0.25) (layer "F.Cu") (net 4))
 (segment (start 70.31 58.49) (end 70.32 58.5) (width 0.25) (layer "F.Cu") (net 4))
 (segment (start 64.3082 57.12) (end 61.62 57.12) (width 0.25) (layer "F.Cu") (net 4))
 (via (at 68.453 58.49) (size 0.6) (drill 0.3) (layers "F.Cu" "B.Cu") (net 4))
 (via (at 65.659 58.4708) (size 0.6) (drill 0.3) (layers "F.Cu" "B.Cu") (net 4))
 (segment (start 68.453 58.49) (end 65.6782 58.49) (width 0.25) (layer "B.Cu") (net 4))
 (segment (start 65.6782 58.49) (end 65.659 58.4708) (width 0.25) (layer "B.Cu") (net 4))
 (segment (start 59.7916 57.2008) (end 59.7408 57.2008) (width 0.25) (layer "F.Cu") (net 3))
 (segment (start 68.472931 59.517669) (end 70.402331 59.517669) (width 0.25) (layer "F.Cu") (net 3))
 (segment (start 68.472931 59.517669) (end 68.4906 59.5) (width 0.25) (layer "F.Cu") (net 3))
 (segment (start 70.402331 59.517669) (end 70.42 59.5) (width 0.25) (layer "F.Cu") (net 3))
 (segment (start 59.7408 57.2008) (end 56.4416 60.5) (width 0.25) (layer "F.Cu") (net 3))
 (segment (start 56.4416 60.5) (end 54.98 60.5) (width 0.25) (layer "F.Cu") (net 3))
 (segment (start 68.472931 59.517669) (end 68.455262 59.5) (width 0.25) (layer "F.Cu") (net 3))
 (segment (start 70.352331 59.517669) (end 70.37 59.5) (width 0.25) (layer "F.Cu") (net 3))
 (via (at 59.7916 57.2008) (size 0.6) (drill 0.3) (layers "F.Cu" "B.Cu") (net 3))
 (via (at 68.472931 59.517669) (size 0.6) (drill 0.3) (layers "F.Cu" "B.Cu") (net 3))
 (segment (start 61.4492 57.2008) (end 59.7916 57.2008) (width 0.25) (layer "B.Cu") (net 3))
 (segment (start 68.472931 59.517669) (end 65.791469 59.517669) (width 0.25) (layer "B.Cu") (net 3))
 (segment (start 65.791469 59.517669) (end 63.4638 57.19) (width 0.25) (layer "B.Cu") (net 3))
 (segment (start 61.46 57.19) (end 61.4492 57.2008) (width 0.25) (layer "B.Cu") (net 3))
 (segment (start 63.4638 57.19) (end 61.46 57.19) (width 0.25) (layer "B.Cu") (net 3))
 (segment (start 63.627 54.4068) (end 63.1698 54.864) (width 0.25) (layer "F.Cu") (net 8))
 (segment (start 64.5202 65.881) (end 64.5202 66.081) (width 0.25) (layer "F.Cu") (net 8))
 (segment (start 62.8402 65.941) (end 62.8452 65.936) (width 0.25) (layer "F.Cu") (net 8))
 (segment (start 63.5452 65.936) (end 64.4652 65.936) (width 0.25) (layer "F.Cu") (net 8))
 (segment (start 61.6202 65.941) (end 60.4038 65.941) (width 0.25) (layer "F.Cu") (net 8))
 (segment (start 65.6082 68.5546) (end 65.1502 68.0966) (width 0.25) (layer "F.Cu") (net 8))
 (segment (start 58.55 65.1) (end 58.55 65.5858) (width 0.25) (layer "F.Cu") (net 8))
 (segment (start 62.8452 65.936) (end 63.5452 65.936) (width 0.25) (layer "F.Cu") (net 8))
 (segment (start 61.727 52.847) (end 62.1942 52.847) (width 0.25) (layer "F.Cu") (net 8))
 (segment (start 68.5546 68.5292) (end 65.6336 68.5292) (width 0.25) (layer "F.Cu") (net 8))
 (segment (start 65.1502 66.711) (end 65.1502 67.481) (width 0.25) (layer "F.Cu") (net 8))
 (segment (start 68.4754 54.6354) (end 68.83 54.99) (width 0.25) (layer "F.Cu") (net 8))
 (segment (start 63.627 53.497) (end 64.1396 53.497) (width 0.25) (layer "F.Cu") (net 8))
 (segment (start 65.278 54.6354) (end 68.4754 54.6354) (width 0.25) (layer "F.Cu") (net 8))
 (segment (start 62.1942 52.847) (end 62.8442 53.497) (width 0.25) (layer "F.Cu") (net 8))
 (segment (start 64.5202 66.081) (end 65.1502 66.711) (width 0.25) (layer "F.Cu") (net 8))
 (segment (start 61.6202 65.941) (end 62.8402 65.941) (width 0.25) (layer "F.Cu") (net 8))
 (segment (start 59.5628 65.1) (end 58.55 65.1) (width 0.25) (layer "F.Cu") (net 8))
 (segment (start 65.6336 68.5292) (end 65.6082 68.5546) (width 0.25) (layer "F.Cu") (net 8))
 (segment (start 63.627 53.497) (end 63.627 54.4068) (width 0.25) (layer "F.Cu") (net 8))
 (segment (start 64.1396 53.497) (end 65.278 54.6354) (width 0.25) (layer "F.Cu") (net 8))
 (segment (start 69.9008 67.183) (end 68.5546 68.5292) (width 0.25) (layer "F.Cu") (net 8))
 (segment (start 60.4038 65.941) (end 59.5628 65.1) (width 0.25) (layer "F.Cu") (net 8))
 (segment (start 69.9008 63.881) (end 69.9008 67.183) (width 0.25) (layer "F.Cu") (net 8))
 (segment (start 62.8442 53.497) (end 63.627 53.497) (width 0.25) (layer "F.Cu") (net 8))
 (segment (start 65.1502 68.0966) (end 65.1502 67.481) (width 0.25) (layer "F.Cu") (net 8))
 (segment (start 64.4652 65.936) (end 64.5202 65.881) (width 0.25) (layer "F.Cu") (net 8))
 (via (at 69.9008 63.881) (size 0.6) (drill 0.3) (layers "F.Cu" "B.Cu") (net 8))
 (via (at 68.83 54.99) (size 0.6) (drill 0.3) (layers "F.Cu" "B.Cu") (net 8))
 (segment (start 69.9008 56.0832) (end 68.83 55.0124) (width 0.25) (layer "B.Cu") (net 8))
 (segment (start 68.83 55.0124) (end 68.83 54.99) (width 0.25) (layer "B.Cu") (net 8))
 (segment (start 69.9008 63.881) (end 69.9008 56.0832) (width 0.25) (layer "B.Cu") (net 8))
 (segment (start 66.7952 63.981) (end 66.7952 63.3544) (width 0.25) (layer "F.Cu") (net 5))
 (segment (start 68.426 63.981) (end 68.4276 63.9826) (width 0.25) (layer "F.Cu") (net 5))
 (segment (start 63.985 59.075) (end 62.7 59.075) (width 0.25) (layer "F.Cu") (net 5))
 (segment (start 66.802 60.932) (end 65.13 59.26) (width 0.25) (layer "F.Cu") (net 5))
 (segment (start 63.825 59.075) (end 62.7 59.075) (width 0.25) (layer "F.Cu") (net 5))
 (segment (start 64.01 59.26) (end 63.825 59.075) (width 0.25) (layer "F.Cu") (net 5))
 (segment (start 66.7952 63.981) (end 68.426 63.981) (width 0.25) (layer "F.Cu") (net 5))
 (segment (start 66.802 63.3476) (end 66.802 60.932) (width 0.25) (layer "F.Cu") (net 5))
 (segment (start 65.13 59.26) (end 64.01 59.26) (width 0.25) (layer "F.Cu") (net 5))
 (segment (start 66.7952 63.3544) (end 66.802 63.3476) (width 0.25) (layer "F.Cu") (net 5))
 (segment (start 62.7 61.66) (end 62.23 62.13) (width 0.25) (layer "F.Cu") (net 9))
 (segment (start 62.23 62.13) (end 57.97 62.13) (width 0.25) (layer "F.Cu") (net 9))
 (segment (start 57.6 62.5) (end 57.6 63.225) (width 0.25) (layer "F.Cu") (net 9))
 (segment (start 62.7 60.925) (end 62.7 61.66) (width 0.25) (layer "F.Cu") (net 9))
 (segment (start 57.97 62.13) (end 57.6 62.5) (width 0.25) (layer "F.Cu") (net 9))
 (segment (start 62.0058 63.225) (end 59.5 63.225) (width 0.25) (layer "F.Cu") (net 7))
 (segment (start 59.545 63.18) (end 59.5 63.225) (width 0.25) (layer "F.Cu") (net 7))
 (segment (start 64.5202 63.981) (end 62.7618 63.981) (width 0.25) (layer "F.Cu") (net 7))
 (segment (start 62.7618 63.981) (end 62.0058 63.225) (width 0.25) (layer "F.Cu") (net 7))
 (segment (start 66.7952 67.346) (end 66.6602 67.481) (width 0.25) (layer "F.Cu") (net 6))
 (segment (start 67.7164 67.3608) (end 68.4276 67.3608) (width 0.25) (layer "F.Cu") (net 6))
 (segment (start 66.7952 65.881) (end 66.7952 67.196) (width 0.25) (layer "F.Cu") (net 6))
 (segment (start 66.5226 67.481) (end 67.5962 67.481) (width 0.25) (layer "F.Cu") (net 6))
 (segment (start 66.5226 67.481) (end 66.1702 67.481) (width 0.25) (layer "F.Cu") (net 6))
 (segment (start 66.7952 67.196) (end 66.7952 67.346) (width 0.25) (layer "F.Cu") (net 6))
 (segment (start 66.6602 67.481) (end 66.5226 67.481) (width 0.25) (layer "F.Cu") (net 6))
 (segment (start 67.5962 67.481) (end 67.7164 67.3608) (width 0.25) (layer "F.Cu") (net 6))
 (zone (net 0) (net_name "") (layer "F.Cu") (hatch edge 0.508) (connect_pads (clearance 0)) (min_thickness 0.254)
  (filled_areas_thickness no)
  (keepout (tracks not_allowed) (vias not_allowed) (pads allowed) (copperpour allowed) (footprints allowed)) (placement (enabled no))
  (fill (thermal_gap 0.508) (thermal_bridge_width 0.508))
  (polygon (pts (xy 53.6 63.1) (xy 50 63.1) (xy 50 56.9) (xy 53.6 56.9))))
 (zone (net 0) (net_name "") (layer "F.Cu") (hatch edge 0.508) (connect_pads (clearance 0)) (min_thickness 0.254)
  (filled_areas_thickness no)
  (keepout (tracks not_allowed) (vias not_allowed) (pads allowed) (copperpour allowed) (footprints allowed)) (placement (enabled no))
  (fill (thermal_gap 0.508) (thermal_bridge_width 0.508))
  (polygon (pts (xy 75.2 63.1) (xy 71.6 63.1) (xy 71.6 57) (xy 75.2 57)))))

